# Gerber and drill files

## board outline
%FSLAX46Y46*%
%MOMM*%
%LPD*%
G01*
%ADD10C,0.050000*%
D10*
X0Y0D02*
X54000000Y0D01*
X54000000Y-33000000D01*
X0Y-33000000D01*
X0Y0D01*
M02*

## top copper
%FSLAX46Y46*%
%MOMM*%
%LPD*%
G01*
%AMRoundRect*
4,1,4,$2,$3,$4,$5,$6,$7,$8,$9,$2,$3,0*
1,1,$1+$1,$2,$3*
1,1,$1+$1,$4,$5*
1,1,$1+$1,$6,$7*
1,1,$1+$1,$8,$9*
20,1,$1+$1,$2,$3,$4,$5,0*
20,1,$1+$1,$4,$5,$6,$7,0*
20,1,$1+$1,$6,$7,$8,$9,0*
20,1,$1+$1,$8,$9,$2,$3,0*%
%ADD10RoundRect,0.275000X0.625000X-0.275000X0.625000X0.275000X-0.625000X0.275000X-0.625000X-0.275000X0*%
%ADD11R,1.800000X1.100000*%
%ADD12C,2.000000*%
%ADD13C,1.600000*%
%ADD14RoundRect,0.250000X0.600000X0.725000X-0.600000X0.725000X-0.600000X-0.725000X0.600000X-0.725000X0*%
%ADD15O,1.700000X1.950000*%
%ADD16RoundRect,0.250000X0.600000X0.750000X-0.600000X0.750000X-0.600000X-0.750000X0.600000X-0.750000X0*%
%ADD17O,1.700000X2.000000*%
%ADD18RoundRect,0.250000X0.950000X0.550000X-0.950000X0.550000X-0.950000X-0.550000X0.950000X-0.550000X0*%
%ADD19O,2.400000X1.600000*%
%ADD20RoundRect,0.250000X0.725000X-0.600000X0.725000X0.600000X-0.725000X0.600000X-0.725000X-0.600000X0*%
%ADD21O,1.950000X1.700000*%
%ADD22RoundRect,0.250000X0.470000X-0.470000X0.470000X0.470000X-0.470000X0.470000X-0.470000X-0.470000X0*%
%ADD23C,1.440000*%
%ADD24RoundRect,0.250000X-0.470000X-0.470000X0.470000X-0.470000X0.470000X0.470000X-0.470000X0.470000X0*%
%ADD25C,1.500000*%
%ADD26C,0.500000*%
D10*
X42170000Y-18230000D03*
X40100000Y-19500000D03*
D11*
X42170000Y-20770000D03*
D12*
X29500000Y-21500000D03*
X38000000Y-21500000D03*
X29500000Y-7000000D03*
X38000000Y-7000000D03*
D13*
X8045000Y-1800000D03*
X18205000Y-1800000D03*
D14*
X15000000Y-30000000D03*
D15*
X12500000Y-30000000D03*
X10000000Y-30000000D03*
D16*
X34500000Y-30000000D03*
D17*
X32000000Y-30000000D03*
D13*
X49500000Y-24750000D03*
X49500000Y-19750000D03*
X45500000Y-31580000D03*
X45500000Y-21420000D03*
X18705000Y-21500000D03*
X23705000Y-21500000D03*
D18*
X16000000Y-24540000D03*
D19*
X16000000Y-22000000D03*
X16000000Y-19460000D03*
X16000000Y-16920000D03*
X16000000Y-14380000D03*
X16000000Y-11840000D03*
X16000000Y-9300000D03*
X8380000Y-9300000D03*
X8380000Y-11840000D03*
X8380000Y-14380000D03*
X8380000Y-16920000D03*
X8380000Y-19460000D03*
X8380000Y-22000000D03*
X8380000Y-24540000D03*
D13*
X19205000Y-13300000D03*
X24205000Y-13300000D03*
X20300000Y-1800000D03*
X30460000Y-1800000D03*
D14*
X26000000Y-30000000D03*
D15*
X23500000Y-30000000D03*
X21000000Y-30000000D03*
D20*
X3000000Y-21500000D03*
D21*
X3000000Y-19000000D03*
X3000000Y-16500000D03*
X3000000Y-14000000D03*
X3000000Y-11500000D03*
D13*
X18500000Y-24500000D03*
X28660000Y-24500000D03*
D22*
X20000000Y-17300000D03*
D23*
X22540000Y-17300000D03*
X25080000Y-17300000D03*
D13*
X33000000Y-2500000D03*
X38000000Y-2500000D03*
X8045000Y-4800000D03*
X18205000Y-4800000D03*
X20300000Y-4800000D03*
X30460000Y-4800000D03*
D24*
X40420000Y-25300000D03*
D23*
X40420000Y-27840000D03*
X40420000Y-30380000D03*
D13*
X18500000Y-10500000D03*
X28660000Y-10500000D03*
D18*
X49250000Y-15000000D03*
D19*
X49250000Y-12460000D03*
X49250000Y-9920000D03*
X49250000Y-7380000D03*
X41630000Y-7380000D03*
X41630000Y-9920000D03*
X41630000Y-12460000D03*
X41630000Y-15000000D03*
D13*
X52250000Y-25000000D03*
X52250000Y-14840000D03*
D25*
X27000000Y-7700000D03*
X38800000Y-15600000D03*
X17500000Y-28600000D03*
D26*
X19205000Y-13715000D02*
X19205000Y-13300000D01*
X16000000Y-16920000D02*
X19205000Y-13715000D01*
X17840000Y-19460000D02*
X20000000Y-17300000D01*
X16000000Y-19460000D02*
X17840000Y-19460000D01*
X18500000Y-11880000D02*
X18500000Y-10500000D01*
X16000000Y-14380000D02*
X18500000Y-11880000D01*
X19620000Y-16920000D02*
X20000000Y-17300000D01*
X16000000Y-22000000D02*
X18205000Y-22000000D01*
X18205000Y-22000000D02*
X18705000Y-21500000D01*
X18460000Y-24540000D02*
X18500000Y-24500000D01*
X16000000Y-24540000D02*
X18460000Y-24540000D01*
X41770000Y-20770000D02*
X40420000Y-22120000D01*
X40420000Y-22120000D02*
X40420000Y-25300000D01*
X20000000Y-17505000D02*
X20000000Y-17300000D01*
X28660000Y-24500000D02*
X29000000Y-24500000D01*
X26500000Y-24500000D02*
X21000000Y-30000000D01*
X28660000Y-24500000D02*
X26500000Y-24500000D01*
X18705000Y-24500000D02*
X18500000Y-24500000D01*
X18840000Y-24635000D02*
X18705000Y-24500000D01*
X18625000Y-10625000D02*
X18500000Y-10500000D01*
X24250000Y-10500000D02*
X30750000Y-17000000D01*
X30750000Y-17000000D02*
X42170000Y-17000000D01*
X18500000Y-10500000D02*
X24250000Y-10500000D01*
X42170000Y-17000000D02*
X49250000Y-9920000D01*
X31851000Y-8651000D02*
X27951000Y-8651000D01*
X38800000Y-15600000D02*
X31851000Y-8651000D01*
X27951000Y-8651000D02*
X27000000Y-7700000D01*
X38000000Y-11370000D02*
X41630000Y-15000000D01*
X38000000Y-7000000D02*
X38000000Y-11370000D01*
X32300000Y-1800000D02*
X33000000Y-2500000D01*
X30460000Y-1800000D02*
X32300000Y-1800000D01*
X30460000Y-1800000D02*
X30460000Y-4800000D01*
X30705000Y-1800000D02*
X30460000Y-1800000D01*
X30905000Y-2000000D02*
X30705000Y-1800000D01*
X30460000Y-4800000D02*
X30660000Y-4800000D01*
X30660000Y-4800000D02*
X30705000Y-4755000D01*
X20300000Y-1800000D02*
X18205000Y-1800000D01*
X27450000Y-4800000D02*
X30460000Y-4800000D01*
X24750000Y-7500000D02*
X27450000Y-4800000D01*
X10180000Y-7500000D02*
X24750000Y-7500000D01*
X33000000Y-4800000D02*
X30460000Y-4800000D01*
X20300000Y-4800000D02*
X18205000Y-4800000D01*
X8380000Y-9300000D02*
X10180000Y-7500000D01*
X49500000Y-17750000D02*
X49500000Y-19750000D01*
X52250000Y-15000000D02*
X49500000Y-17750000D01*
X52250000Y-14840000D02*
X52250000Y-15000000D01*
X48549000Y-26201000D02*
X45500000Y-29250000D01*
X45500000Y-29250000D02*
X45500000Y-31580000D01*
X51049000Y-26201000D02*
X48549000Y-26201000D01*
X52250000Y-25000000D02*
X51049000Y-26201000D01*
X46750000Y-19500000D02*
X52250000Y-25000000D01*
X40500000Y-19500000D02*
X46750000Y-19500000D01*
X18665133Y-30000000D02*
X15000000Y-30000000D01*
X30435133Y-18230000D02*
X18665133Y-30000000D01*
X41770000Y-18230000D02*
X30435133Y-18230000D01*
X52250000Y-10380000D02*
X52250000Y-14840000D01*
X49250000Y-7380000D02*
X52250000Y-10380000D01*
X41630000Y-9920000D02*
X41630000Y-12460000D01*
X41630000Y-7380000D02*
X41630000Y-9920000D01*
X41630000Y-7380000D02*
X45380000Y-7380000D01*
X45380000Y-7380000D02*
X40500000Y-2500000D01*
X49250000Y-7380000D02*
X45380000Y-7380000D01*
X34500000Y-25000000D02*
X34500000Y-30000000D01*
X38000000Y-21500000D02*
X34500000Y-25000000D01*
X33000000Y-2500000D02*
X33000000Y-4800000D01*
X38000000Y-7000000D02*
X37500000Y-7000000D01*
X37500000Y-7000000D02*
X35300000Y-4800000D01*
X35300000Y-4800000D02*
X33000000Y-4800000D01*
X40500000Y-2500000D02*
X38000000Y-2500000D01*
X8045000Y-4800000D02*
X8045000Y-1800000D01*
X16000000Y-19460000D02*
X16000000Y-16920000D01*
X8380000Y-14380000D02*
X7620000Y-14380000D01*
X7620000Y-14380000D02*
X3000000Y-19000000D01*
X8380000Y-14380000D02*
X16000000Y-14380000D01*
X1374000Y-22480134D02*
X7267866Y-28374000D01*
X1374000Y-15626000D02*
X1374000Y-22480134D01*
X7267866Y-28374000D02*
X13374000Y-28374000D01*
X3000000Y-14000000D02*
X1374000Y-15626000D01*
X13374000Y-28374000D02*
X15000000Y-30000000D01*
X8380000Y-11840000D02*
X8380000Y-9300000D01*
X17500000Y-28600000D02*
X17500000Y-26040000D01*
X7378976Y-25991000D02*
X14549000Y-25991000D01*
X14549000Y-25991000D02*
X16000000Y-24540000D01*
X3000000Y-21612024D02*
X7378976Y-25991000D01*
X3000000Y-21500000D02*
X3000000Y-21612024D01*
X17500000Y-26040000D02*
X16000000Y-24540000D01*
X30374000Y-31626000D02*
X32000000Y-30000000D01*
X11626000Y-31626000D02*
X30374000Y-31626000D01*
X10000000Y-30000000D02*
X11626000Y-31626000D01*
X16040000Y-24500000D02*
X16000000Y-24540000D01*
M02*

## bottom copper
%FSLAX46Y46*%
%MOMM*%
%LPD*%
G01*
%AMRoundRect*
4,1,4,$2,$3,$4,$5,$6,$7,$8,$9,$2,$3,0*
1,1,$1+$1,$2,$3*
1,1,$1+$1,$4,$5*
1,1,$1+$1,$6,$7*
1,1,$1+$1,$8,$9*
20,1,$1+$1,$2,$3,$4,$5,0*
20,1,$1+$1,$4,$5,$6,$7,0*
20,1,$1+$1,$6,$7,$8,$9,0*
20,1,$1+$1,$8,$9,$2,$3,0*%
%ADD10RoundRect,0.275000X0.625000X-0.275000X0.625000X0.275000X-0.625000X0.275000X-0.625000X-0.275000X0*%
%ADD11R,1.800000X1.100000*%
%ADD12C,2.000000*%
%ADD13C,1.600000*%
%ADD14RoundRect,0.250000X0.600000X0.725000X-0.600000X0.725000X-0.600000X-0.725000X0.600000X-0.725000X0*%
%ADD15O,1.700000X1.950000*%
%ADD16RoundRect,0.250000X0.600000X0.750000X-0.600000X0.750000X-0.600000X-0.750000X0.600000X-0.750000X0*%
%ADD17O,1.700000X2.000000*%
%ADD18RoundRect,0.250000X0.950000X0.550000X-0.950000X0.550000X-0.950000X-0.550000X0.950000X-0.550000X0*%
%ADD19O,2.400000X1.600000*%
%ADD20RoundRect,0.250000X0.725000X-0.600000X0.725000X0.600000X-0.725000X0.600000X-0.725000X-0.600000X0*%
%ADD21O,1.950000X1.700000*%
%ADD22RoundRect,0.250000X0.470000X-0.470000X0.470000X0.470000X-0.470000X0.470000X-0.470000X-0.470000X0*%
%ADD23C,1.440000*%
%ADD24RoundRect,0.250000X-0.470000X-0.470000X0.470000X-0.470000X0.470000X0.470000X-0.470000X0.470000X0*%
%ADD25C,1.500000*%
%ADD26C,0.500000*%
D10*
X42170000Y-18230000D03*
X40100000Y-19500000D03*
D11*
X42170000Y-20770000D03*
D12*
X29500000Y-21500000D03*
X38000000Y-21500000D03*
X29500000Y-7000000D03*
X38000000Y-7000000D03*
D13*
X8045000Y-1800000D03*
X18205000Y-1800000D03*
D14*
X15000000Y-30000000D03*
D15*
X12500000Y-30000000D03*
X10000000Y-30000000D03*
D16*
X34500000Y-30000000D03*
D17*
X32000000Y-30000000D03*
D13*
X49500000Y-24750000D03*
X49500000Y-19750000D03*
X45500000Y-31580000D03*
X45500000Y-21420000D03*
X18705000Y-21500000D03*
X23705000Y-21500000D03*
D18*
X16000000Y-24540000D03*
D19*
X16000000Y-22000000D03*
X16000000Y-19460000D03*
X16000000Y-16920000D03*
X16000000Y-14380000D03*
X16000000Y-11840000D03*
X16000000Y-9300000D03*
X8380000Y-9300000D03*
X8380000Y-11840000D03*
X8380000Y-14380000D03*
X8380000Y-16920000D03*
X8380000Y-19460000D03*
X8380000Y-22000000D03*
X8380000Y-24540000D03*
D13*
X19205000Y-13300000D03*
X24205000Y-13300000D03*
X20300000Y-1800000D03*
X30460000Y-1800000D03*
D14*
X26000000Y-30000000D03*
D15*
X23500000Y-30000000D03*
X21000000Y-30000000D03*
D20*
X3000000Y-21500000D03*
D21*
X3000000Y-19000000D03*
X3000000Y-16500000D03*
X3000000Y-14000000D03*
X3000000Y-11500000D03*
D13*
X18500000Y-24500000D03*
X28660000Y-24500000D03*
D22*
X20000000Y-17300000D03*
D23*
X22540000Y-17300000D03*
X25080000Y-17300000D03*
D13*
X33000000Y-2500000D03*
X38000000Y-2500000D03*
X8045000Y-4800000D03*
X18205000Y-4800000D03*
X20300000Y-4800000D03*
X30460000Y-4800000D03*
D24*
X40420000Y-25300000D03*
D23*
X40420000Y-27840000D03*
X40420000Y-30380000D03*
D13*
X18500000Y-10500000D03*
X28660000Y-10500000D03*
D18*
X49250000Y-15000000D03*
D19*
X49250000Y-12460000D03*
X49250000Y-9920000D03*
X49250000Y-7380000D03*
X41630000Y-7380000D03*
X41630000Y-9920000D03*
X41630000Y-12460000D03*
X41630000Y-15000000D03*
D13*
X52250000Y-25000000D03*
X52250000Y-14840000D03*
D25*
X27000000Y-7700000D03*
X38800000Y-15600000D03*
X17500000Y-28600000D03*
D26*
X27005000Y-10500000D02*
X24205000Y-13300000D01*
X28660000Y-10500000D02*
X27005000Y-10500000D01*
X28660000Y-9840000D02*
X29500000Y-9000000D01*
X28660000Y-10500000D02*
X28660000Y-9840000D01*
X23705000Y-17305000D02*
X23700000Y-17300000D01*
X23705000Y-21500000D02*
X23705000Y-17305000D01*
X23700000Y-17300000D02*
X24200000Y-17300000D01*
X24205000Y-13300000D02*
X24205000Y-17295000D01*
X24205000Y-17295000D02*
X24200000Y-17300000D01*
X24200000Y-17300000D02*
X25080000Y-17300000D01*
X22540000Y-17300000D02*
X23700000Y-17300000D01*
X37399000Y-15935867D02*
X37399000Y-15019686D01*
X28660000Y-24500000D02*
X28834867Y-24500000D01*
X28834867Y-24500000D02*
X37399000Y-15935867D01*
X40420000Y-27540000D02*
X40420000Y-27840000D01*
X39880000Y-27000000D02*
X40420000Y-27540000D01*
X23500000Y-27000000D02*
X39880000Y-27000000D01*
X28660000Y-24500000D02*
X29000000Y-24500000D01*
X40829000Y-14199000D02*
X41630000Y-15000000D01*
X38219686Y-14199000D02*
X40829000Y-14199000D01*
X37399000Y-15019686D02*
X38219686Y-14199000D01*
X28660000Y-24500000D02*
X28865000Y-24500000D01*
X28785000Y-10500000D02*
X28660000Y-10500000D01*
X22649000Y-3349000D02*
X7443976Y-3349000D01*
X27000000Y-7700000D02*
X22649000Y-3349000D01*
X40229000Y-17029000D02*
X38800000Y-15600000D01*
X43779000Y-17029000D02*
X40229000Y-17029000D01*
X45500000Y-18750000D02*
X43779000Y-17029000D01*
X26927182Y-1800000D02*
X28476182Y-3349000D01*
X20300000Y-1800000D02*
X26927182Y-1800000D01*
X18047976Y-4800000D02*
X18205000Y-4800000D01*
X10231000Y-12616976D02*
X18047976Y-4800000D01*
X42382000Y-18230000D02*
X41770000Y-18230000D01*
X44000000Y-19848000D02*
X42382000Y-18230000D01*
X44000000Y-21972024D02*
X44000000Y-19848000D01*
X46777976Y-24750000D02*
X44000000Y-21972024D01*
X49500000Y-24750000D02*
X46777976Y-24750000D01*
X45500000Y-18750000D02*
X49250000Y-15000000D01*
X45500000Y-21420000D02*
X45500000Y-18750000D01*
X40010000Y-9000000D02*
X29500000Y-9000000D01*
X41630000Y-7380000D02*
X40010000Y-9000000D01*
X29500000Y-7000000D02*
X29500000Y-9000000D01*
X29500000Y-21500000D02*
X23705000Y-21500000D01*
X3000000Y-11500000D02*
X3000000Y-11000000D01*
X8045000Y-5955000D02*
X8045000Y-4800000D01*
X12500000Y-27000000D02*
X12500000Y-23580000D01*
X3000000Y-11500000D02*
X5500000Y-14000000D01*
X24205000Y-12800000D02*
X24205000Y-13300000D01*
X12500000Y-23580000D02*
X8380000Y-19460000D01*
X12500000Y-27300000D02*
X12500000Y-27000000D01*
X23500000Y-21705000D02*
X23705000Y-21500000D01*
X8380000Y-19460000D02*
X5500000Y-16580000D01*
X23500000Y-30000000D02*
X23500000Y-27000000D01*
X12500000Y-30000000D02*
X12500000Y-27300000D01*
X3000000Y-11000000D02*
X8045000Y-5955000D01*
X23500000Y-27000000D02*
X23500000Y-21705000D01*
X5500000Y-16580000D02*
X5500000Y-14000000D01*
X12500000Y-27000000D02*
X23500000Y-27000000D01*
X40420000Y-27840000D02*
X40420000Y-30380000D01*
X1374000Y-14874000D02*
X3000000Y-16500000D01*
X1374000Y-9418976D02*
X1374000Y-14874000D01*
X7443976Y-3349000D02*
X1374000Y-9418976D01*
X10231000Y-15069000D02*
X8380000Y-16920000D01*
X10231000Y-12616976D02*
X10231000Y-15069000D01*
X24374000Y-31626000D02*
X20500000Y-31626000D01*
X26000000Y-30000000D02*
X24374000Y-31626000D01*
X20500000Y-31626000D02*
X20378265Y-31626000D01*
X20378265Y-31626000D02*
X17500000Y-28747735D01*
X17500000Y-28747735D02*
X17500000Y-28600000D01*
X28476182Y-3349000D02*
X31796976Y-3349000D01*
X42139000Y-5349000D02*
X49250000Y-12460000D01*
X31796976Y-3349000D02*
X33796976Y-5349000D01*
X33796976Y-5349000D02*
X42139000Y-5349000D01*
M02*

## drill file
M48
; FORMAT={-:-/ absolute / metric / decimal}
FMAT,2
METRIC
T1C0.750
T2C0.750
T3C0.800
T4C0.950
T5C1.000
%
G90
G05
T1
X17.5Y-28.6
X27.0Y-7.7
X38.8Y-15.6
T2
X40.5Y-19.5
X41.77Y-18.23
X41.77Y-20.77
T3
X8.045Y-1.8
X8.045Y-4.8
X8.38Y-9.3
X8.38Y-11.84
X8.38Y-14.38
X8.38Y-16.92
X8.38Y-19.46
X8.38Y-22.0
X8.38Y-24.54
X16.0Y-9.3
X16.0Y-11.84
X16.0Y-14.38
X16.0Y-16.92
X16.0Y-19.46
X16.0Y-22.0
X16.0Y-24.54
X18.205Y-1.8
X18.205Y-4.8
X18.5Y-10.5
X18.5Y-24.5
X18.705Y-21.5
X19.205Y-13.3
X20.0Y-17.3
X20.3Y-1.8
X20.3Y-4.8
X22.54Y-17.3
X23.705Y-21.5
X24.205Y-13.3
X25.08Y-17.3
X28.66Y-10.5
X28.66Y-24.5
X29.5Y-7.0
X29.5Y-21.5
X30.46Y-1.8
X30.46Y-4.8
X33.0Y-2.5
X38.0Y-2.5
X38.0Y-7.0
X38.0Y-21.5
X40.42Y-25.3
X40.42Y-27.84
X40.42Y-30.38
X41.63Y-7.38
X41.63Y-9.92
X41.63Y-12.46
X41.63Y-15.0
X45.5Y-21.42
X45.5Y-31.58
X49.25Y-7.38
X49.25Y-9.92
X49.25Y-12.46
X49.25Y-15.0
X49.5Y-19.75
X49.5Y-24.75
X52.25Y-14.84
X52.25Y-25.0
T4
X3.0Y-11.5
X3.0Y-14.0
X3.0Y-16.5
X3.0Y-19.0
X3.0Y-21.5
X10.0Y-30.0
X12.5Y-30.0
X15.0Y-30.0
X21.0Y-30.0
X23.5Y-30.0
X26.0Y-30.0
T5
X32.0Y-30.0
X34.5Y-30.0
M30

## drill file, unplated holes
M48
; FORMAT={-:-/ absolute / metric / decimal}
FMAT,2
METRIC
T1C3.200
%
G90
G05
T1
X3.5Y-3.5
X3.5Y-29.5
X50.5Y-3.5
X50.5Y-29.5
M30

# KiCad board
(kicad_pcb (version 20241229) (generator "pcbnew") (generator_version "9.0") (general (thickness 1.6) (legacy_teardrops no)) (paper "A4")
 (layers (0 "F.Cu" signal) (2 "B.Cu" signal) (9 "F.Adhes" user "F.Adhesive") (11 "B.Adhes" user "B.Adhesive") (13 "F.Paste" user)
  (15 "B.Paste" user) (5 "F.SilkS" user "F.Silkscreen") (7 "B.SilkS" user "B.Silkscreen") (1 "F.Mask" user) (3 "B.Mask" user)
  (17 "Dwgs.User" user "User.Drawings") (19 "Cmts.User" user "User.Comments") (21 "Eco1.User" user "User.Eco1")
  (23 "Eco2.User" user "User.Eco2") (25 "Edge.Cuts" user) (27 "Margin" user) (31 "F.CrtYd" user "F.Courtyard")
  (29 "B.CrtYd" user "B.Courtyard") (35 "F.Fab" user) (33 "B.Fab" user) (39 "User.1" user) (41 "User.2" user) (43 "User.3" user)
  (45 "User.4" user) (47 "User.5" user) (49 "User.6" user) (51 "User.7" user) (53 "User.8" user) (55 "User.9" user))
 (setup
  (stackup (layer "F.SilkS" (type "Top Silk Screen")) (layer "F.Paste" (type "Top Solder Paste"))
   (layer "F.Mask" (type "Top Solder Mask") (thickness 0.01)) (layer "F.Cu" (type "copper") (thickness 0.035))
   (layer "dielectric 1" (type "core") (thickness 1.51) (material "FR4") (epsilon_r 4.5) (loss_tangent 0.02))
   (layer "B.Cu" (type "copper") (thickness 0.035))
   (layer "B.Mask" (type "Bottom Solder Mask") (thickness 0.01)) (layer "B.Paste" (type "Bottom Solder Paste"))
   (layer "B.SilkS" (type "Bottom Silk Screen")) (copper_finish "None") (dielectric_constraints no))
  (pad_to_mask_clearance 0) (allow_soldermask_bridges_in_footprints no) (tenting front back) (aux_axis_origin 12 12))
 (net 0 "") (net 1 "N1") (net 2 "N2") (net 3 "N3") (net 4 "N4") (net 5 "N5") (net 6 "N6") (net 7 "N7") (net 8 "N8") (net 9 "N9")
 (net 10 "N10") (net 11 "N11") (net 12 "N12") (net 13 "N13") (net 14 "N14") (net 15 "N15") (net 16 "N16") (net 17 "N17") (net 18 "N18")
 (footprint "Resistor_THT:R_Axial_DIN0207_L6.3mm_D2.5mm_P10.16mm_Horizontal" (layer "F.Cu") (at 20.045 13.8)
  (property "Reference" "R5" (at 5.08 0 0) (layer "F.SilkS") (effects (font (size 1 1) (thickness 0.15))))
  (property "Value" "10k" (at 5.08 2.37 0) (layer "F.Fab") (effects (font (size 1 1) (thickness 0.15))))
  (pad "1" thru_hole circle (at 0 0) (size 1.6 1.6) (drill 0.8) (layers "*.Cu" "*.Mask") (remove_unused_layers no) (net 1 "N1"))
  (pad "2" thru_hole circle (at 10.16 0) (size 1.6 1.6) (drill 0.8) (layers "*.Cu" "*.Mask") (remove_unused_layers no) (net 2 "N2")))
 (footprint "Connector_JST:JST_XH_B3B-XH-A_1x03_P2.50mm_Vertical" (layer "F.Cu") (at 27 42 180)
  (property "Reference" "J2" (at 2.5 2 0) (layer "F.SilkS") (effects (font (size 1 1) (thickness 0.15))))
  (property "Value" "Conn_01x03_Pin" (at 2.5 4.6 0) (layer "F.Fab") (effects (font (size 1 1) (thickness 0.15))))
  (pad "1" thru_hole roundrect (at 0 0 180) (size 1.7 1.95) (drill 0.95) (layers "*.Cu" "*.Mask") (remove_unused_layers no)
   (roundrect_rratio 0.147059) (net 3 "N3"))
  (pad "2" thru_hole oval (at 2.5 0 180) (size 1.7 1.95) (drill 0.95) (layers "*.Cu" "*.Mask") (remove_unused_layers no) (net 1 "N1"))
  (pad "3" thru_hole oval (at 5 0 180) (size 1.7 1.95) (drill 0.95) (layers "*.Cu" "*.Mask") (remove_unused_layers no) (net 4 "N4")))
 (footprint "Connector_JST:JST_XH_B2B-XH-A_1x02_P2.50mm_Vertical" (layer "F.Cu") (at 46.5 42 180)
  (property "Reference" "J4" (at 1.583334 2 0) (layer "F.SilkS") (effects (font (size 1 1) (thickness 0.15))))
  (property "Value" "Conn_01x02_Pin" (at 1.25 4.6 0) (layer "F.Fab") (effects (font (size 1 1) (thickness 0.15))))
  (pad "1" thru_hole roundrect (at 0 0 180) (size 1.7 2) (drill 1) (layers "*.Cu" "*.Mask") (remove_unused_layers no)
   (roundrect_rratio 0.147059) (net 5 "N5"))
  (pad "2" thru_hole oval (at 2.5 0 180) (size 1.7 2) (drill 1) (layers "*.Cu" "*.Mask") (remove_unused_layers no) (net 4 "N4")))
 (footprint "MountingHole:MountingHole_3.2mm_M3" (layer "F.Cu") (at 15.5 41.5 90)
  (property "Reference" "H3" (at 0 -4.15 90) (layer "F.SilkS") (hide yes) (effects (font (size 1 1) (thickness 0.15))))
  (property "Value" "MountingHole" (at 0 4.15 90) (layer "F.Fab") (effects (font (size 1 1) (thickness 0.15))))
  (pad "" np_thru_hole circle (at 0 0 90) (size 3.2 3.2) (drill 3.2) (layers "*.Cu" "*.Mask")))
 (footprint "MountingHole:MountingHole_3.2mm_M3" (layer "F.Cu") (at 62.5 15.5 90)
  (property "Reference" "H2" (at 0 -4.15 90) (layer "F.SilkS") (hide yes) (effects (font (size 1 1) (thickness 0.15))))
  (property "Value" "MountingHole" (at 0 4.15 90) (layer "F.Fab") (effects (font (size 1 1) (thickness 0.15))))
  (pad "" np_thru_hole circle (at 0 0 90) (size 3.2 3.2) (drill 3.2) (layers "*.Cu" "*.Mask")))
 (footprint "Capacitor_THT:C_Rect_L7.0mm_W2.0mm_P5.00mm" (layer "F.Cu") (at 61.5 36.75 90)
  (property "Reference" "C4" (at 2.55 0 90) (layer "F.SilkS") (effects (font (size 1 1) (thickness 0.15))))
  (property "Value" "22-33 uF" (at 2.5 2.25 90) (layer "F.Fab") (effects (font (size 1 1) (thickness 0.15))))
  (pad "1" thru_hole circle (at 0 0 90) (size 1.6 1.6) (drill 0.8) (layers "*.Cu" "*.Mask") (remove_unused_layers no) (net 3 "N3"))
  (pad "2" thru_hole circle (at 5 0 90) (size 1.6 1.6) (drill 0.8) (layers "*.Cu" "*.Mask") (remove_unused_layers no) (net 1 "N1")))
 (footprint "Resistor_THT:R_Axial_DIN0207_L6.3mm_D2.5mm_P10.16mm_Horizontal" (layer "F.Cu") (at 57.5 43.58 90)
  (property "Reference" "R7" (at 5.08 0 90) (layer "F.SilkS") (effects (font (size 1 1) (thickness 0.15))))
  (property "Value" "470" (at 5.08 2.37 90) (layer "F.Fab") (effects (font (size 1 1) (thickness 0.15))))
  (pad "1" thru_hole circle (at 0 0 90) (size 1.6 1.6) (drill 0.8) (layers "*.Cu" "*.Mask") (remove_unused_layers no) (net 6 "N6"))
  (pad "2" thru_hole circle (at 10.16 0 90) (size 1.6 1.6) (drill 0.8) (layers "*.Cu" "*.Mask") (remove_unused_layers no) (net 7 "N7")))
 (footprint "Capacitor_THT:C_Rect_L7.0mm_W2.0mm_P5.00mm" (layer "F.Cu") (at 30.705 33.5)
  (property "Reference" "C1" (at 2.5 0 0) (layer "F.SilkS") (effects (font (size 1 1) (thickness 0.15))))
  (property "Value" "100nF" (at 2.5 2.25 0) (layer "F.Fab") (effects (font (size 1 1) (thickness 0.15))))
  (pad "1" thru_hole circle (at 0 0) (size 1.6 1.6) (drill 0.8) (layers "*.Cu" "*.Mask") (remove_unused_layers no) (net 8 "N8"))
  (pad "2" thru_hole circle (at 5 0) (size 1.6 1.6) (drill 0.8) (layers "*.Cu" "*.Mask") (remove_unused_layers no) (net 1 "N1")))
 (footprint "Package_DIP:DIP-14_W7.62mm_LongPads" (layer "F.Cu") (at 28 36.54 180)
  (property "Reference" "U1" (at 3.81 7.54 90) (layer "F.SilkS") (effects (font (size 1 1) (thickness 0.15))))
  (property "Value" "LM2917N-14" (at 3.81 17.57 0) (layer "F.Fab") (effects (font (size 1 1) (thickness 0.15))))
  (pad "1" thru_hole roundrect (at 0 0 180) (size 2.4 1.6) (drill 0.8) (layers "*.Cu" "*.Mask") (remove_unused_layers no)
   (roundrect_rratio 0.15625) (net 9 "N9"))
  (pad "2" thru_hole oval (at 0 2.54 180) (size 2.4 1.6) (drill 0.8) (layers "*.Cu" "*.Mask") (remove_unused_layers no) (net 8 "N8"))
  (pad "3" thru_hole oval (at 0 5.08 180) (size 2.4 1.6) (drill 0.8) (layers "*.Cu" "*.Mask") (remove_unused_layers no) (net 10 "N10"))
  (pad "4" thru_hole oval (at 0 7.62 180) (size 2.4 1.6) (drill 0.8) (layers "*.Cu" "*.Mask") (remove_unused_layers no) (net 10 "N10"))
  (pad "5" thru_hole oval (at 0 10.16 180) (size 2.4 1.6) (drill 0.8) (layers "*.Cu" "*.Mask") (remove_unused_layers no) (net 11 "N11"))
  (pad "6" thru_hole oval (at 0 12.7 180) (size 2.4 1.6) (drill 0.8) (layers "*.Cu" "*.Mask") (remove_unused_layers no) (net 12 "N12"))
  (pad "7" thru_hole oval (at 0 15.24 180) (size 2.4 1.6) (drill 0.8) (layers "*.Cu" "*.Mask") (remove_unused_layers no) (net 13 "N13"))
  (pad "8" thru_hole oval (at 7.62 15.24 180) (size 2.4 1.6) (drill 0.8) (layers "*.Cu" "*.Mask") (remove_unused_layers no) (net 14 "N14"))
  (pad "9" thru_hole oval (at 7.62 12.7 180) (size 2.4 1.6) (drill 0.8) (layers "*.Cu" "*.Mask") (remove_unused_layers no) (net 14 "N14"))
  (pad "10" thru_hole oval (at 7.62 10.16 180) (size 2.4 1.6) (drill 0.8) (layers "*.Cu" "*.Mask") (remove_unused_layers no) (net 11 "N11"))
  (pad "11" thru_hole oval (at 7.62 7.62 180) (size 2.4 1.6) (drill 0.8) (layers "*.Cu" "*.Mask") (remove_unused_layers no) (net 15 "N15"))
  (pad "12" thru_hole oval (at 7.62 5.08 180) (size 2.4 1.6) (drill 0.8) (layers "*.Cu" "*.Mask") (remove_unused_layers no) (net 1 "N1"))
  (pad "13" thru_hole oval (at 7.62 2.54 180) (size 2.4 1.6) (drill 0.8) (layers "*.Cu" "*.Mask") (remove_unused_layers no) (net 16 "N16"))
  (pad "14" thru_hole oval (at 7.62 0 180) (size 2.4 1.6) (drill 0.8) (layers "*.Cu" "*.Mask") (remove_unused_layers no) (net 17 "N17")))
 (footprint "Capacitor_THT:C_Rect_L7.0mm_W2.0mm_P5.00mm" (layer "F.Cu") (at 31.205 25.3)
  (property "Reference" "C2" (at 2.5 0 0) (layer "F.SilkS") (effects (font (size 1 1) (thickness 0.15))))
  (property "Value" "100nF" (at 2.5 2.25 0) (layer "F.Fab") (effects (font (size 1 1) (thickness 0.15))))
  (pad "1" thru_hole circle (at 0 0) (size 1.6 1.6) (drill 0.8) (layers "*.Cu" "*.Mask") (remove_unused_layers no) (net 10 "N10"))
  (pad "2" thru_hole circle (at 5 0) (size 1.6 1.6) (drill 0.8) (layers "*.Cu" "*.Mask") (remove_unused_layers no) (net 1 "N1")))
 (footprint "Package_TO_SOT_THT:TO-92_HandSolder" (layer "F.Cu") (at 53.77 32.77 90)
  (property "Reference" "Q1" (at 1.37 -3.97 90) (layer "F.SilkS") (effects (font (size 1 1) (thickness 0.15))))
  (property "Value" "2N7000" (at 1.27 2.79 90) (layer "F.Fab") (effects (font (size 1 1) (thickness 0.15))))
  (pad "1" thru_hole rect (at 0 0 90) (size 1.1 1.8) (drill 0.75 (offset 0 0.4)) (layers "*.Cu" "*.Mask") (remove_unused_layers no)
   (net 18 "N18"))
  (pad "2" thru_hole roundrect (at 1.27 -1.27 90) (size 1.1 1.8) (drill 0.75 (offset 0 -0.4)) (layers "*.Cu" "*.Mask")
   (remove_unused_layers no) (roundrect_rratio 0.25) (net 6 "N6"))
  (pad "3" thru_hole roundrect (at 2.54 0 90) (size 1.1 1.8) (drill 0.75 (offset 0 0.4)) (layers "*.Cu" "*.Mask") (remove_unused_layers no)
   (roundrect_rratio 0.25) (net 3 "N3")))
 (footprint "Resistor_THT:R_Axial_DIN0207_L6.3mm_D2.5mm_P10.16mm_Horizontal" (layer "F.Cu") (at 32.3 13.8)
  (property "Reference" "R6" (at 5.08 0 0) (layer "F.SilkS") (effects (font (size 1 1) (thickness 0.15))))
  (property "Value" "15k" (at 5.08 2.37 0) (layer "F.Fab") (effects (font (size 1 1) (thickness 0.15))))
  (pad "1" thru_hole circle (at 0 0) (size 1.6 1.6) (drill 0.8) (layers "*.Cu" "*.Mask") (remove_unused_layers no) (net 2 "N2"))
  (pad "2" thru_hole circle (at 10.16 0) (size 1.6 1.6) (drill 0.8) (layers "*.Cu" "*.Mask") (remove_unused_layers no) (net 14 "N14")))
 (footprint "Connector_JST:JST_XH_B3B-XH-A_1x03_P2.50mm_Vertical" (layer "F.Cu") (at 38 42 180)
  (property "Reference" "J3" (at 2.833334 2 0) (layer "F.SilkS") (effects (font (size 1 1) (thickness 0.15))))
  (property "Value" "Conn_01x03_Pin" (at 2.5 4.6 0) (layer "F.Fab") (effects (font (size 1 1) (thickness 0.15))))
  (pad "1" thru_hole roundrect (at 0 0 180) (size 1.7 1.95) (drill 0.95) (layers "*.Cu" "*.Mask") (remove_unused_layers no)
   (roundrect_rratio 0.147059) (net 9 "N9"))
  (pad "2" thru_hole oval (at 2.5 0 180) (size 1.7 1.95) (drill 0.95) (layers "*.Cu" "*.Mask") (remove_unused_layers no) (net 1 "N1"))
  (pad "3" thru_hole oval (at 5 0 180) (size 1.7 1.95) (drill 0.95) (layers "*.Cu" "*.Mask") (remove_unused_layers no) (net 14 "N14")))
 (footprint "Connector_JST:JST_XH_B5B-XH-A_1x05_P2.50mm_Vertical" (layer "F.Cu") (at 15 33.5 90)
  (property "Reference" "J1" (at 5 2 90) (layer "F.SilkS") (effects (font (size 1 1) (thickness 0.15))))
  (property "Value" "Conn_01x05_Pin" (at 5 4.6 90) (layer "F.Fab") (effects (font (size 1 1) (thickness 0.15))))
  (pad "1" thru_hole roundrect (at 0 0 90) (size 1.7 1.95) (drill 0.95) (layers "*.Cu" "*.Mask") (remove_unused_layers no)
   (roundrect_rratio 0.147059) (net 9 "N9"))
  (pad "2" thru_hole oval (at 2.5 0 90) (size 1.7 1.95) (drill 0.95) (layers "*.Cu" "*.Mask") (remove_unused_layers no) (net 11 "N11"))
  (pad "3" thru_hole oval (at 5 0 90) (size 1.7 1.95) (drill 0.95) (layers "*.Cu" "*.Mask") (remove_unused_layers no) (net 7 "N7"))
  (pad "4" thru_hole oval (at 7.5 0 90) (size 1.7 1.95) (drill 0.95) (layers "*.Cu" "*.Mask") (remove_unused_layers no) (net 3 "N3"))
  (pad "5" thru_hole oval (at 10 0 90) (size 1.7 1.95) (drill 0.95) (layers "*.Cu" "*.Mask") (remove_unused_layers no) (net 1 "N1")))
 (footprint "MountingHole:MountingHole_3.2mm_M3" (layer "F.Cu") (at 62.5 41.5 90)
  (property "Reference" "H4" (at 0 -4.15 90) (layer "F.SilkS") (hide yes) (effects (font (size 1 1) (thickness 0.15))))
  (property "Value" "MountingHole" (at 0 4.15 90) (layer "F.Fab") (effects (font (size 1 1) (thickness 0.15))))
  (pad "" np_thru_hole circle (at 0 0 90) (size 3.2 3.2) (drill 3.2) (layers "*.Cu" "*.Mask")))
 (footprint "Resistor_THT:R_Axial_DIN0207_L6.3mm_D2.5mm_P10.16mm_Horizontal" (layer "F.Cu") (at 30.5 36.5)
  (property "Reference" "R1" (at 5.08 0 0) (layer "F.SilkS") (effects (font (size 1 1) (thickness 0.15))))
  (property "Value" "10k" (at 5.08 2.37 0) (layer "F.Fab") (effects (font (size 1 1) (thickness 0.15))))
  (pad "1" thru_hole circle (at 0 0) (size 1.6 1.6) (drill 0.8) (layers "*.Cu" "*.Mask") (remove_unused_layers no) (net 9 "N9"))
  (pad "2" thru_hole circle (at 10.16 0) (size 1.6 1.6) (drill 0.8) (layers "*.Cu" "*.Mask") (remove_unused_layers no) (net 14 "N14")))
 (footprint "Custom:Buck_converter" (layer "F.Cu") (at 45.75 26.25 90)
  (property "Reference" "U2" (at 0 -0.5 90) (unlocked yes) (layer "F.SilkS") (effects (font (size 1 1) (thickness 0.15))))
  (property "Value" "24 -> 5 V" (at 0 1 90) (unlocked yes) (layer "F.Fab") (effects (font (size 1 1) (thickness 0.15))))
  (pad "1" thru_hole circle (at -7.25 -4.25 90) (size 2 2) (drill 0.8) (layers "*.Cu" "*.Mask") (remove_unused_layers no) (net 1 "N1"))
  (pad "2" thru_hole circle (at -7.25 4.25 90) (size 2 2) (drill 0.8) (layers "*.Cu" "*.Mask") (remove_unused_layers no) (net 5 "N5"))
  (pad "3" thru_hole circle (at 7.25 -4.25 90) (size 2 2) (drill 0.8) (layers "*.Cu" "*.Mask") (remove_unused_layers no) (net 1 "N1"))
  (pad "4" thru_hole circle (at 7.25 4.25 90) (size 2 2) (drill 0.8) (layers "*.Cu" "*.Mask") (remove_unused_layers no) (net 14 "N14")))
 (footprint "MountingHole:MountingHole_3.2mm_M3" (layer "F.Cu") (at 15.5 15.5 90)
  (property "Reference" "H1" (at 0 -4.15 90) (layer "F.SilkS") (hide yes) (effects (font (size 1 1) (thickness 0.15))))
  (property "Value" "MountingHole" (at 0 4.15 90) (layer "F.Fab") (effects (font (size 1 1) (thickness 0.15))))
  (pad "" np_thru_hole circle (at 0 0 90) (size 3.2 3.2) (drill 3.2) (layers "*.Cu" "*.Mask")))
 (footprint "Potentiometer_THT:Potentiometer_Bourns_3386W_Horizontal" (layer "F.Cu") (at 32 29.3)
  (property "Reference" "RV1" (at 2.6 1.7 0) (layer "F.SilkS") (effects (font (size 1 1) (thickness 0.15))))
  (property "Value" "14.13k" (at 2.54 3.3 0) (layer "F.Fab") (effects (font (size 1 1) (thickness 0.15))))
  (pad "1" thru_hole roundrect (at 0 0 90) (size 1.44 1.44) (drill 0.8) (layers "*.Cu" "*.Mask") (remove_unused_layers no)
   (roundrect_rratio 0.1736111111) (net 10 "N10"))
  (pad "2" thru_hole circle (at 2.54 0 90) (size 1.44 1.44) (drill 0.8) (layers "*.Cu" "*.Mask") (remove_unused_layers no) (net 1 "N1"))
  (pad "3" thru_hole circle (at 5.08 0 90) (size 1.44 1.44) (drill 0.8) (layers "*.Cu" "*.Mask") (remove_unused_layers no) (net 1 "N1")))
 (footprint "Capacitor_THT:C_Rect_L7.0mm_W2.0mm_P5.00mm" (layer "F.Cu") (at 45 14.5)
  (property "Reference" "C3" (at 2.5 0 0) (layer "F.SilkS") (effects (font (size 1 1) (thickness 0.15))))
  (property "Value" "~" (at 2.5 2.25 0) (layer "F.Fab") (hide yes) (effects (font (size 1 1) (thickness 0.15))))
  (pad "1" thru_hole circle (at 0 0) (size 1.6 1.6) (drill 0.8) (layers "*.Cu" "*.Mask") (remove_unused_layers no) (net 14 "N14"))
  (pad "2" thru_hole circle (at 5 0) (size 1.6 1.6) (drill 0.8) (layers "*.Cu" "*.Mask") (remove_unused_layers no) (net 1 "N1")))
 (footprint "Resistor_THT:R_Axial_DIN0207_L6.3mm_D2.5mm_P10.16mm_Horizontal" (layer "F.Cu") (at 20.045 16.8)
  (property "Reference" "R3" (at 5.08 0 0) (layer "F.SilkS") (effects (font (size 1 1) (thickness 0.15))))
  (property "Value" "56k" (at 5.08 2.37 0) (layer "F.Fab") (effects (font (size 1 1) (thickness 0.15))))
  (pad "1" thru_hole circle (at 0 0) (size 1.6 1.6) (drill 0.8) (layers "*.Cu" "*.Mask") (remove_unused_layers no) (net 1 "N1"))
  (pad "2" thru_hole circle (at 10.16 0) (size 1.6 1.6) (drill 0.8) (layers "*.Cu" "*.Mask") (remove_unused_layers no) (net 15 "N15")))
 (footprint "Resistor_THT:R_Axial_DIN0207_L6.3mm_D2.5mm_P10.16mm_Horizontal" (layer "F.Cu") (at 32.3 16.8)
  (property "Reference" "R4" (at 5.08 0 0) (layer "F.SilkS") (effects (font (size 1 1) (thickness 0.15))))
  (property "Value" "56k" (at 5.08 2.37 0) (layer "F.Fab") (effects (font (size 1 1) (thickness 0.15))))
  (pad "1" thru_hole circle (at 0 0) (size 1.6 1.6) (drill 0.8) (layers "*.Cu" "*.Mask") (remove_unused_layers no) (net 15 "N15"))
  (pad "2" thru_hole circle (at 10.16 0) (size 1.6 1.6) (drill 0.8) (layers "*.Cu" "*.Mask") (remove_unused_layers no) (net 14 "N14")))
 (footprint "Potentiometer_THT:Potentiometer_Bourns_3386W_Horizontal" (layer "F.Cu") (at 52.42 37.3 -90)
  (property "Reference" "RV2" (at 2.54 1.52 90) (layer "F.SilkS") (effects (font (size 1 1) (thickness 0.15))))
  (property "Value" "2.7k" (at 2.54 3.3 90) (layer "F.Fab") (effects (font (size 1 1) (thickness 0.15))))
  (pad "1" thru_hole roundrect (at 0 0) (size 1.44 1.44) (drill 0.8) (layers "*.Cu" "*.Mask") (remove_unused_layers no)
   (roundrect_rratio 0.1736111111) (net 18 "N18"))
  (pad "2" thru_hole circle (at 2.54 0) (size 1.44 1.44) (drill 0.8) (layers "*.Cu" "*.Mask") (remove_unused_layers no) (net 1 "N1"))
  (pad "3" thru_hole circle (at 5.08 0) (size 1.44 1.44) (drill 0.8) (layers "*.Cu" "*.Mask") (remove_unused_layers no) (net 1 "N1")))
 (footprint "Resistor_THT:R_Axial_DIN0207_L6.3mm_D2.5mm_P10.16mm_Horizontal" (layer "F.Cu") (at 30.5 22.5)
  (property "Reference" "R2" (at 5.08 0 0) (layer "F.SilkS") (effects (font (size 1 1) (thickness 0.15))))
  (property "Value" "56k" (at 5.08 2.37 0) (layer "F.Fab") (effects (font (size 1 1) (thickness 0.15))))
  (pad "1" thru_hole circle (at 0 0) (size 1.6 1.6) (drill 0.8) (layers "*.Cu" "*.Mask") (remove_unused_layers no) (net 11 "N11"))
  (pad "2" thru_hole circle (at 10.16 0) (size 1.6 1.6) (drill 0.8) (layers "*.Cu" "*.Mask") (remove_unused_layers no) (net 1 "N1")))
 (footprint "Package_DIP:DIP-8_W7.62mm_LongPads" (layer "F.Cu") (at 61.25 27 180)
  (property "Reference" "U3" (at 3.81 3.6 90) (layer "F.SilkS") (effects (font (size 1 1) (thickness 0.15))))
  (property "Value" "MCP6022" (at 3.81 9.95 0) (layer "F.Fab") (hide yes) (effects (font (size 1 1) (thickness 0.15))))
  (pad "1" thru_hole roundrect (at 0 0 180) (size 2.4 1.6) (drill 0.8) (layers "*.Cu" "*.Mask") (remove_unused_layers no)
   (roundrect_rratio 0.15625) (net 7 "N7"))
  (pad "2" thru_hole oval (at 0 2.54 180) (size 2.4 1.6) (drill 0.8) (layers "*.Cu" "*.Mask") (remove_unused_layers no) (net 2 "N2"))
  (pad "3" thru_hole oval (at 0 5.08 180) (size 2.4 1.6) (drill 0.8) (layers "*.Cu" "*.Mask") (remove_unused_layers no) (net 11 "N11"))
  (pad "4" thru_hole oval (at 0 7.62 180) (size 2.4 1.6) (drill 0.8) (layers "*.Cu" "*.Mask") (remove_unused_layers no) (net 1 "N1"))
  (pad "5" thru_hole oval (at 7.62 7.62 180) (size 2.4 1.6) (drill 0.8) (layers "*.Cu" "*.Mask") (remove_unused_layers no) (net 1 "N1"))
  (pad "6" thru_hole oval (at 7.62 5.08 180) (size 2.4 1.6) (drill 0.8) (layers "*.Cu" "*.Mask") (remove_unused_layers no) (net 1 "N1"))
  (pad "7" thru_hole oval (at 7.62 2.54 180) (size 2.4 1.6) (drill 0.8) (layers "*.Cu" "*.Mask") (remove_unused_layers no) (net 1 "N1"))
  (pad "8" thru_hole oval (at 7.62 0 180) (size 2.4 1.6) (drill 0.8) (layers "*.Cu" "*.Mask") (remove_unused_layers no) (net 14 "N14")))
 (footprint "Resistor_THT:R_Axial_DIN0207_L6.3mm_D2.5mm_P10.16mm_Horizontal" (layer "F.Cu") (at 64.25 37 90)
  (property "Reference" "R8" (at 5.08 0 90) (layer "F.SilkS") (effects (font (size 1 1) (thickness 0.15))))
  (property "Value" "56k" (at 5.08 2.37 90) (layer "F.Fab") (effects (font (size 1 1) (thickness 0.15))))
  (pad "1" thru_hole circle (at 0 0 90) (size 1.6 1.6) (drill 0.8) (layers "*.Cu" "*.Mask") (remove_unused_layers no) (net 6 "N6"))
  (pad "2" thru_hole circle (at 10.16 0 90) (size 1.6 1.6) (drill 0.8) (layers "*.Cu" "*.Mask") (remove_unused_layers no) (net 1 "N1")))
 (gr_rect (start 12 12) (end 66 45) (stroke (width 0.05) (type default)) (fill no) (layer "Edge.Cuts"))
 (segment (start 28 34) (end 30.205 34) (width 0.5) (layer "F.Cu") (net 8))
 (segment (start 30.205 34) (end 30.705 33.5) (width 0.5) (layer "F.Cu") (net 8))
 (segment (start 28 31.46) (end 29.84 31.46) (width 0.5) (layer "F.Cu") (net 10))
 (segment (start 32 29.505) (end 32 29.3) (width 0.5) (layer "F.Cu") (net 10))
 (segment (start 31.62 28.92) (end 32 29.3) (width 0.5) (layer "F.Cu") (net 10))
 (segment (start 28 28.92) (end 31.205 25.715) (width 0.5) (layer "F.Cu") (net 10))
 (segment (start 31.205 25.715) (end 31.205 25.3) (width 0.5) (layer "F.Cu") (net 10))
 (segment (start 28 31.46) (end 28 28.92) (width 0.5) (layer "F.Cu") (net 10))
 (segment (start 29.84 31.46) (end 32 29.3) (width 0.5) (layer "F.Cu") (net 10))
 (segment (start 30.625 22.625) (end 30.5 22.5) (width 0.5) (layer "F.Cu") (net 11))
 (segment (start 42.75 29) (end 54.17 29) (width 0.5) (layer "F.Cu") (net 11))
 (segment (start 28 26.38) (end 30.5 23.88) (width 0.5) (layer "F.Cu") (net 11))
 (segment (start 20.38 26.38) (end 19.62 26.38) (width 0.5) (layer "F.Cu") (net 11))
 (segment (start 30.5 22.5) (end 36.25 22.5) (width 0.5) (layer "F.Cu") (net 11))
 (segment (start 19.62 26.38) (end 15 31) (width 0.5) (layer "F.Cu") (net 11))
 (segment (start 36.25 22.5) (end 42.75 29) (width 0.5) (layer "F.Cu") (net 11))
 (segment (start 54.17 29) (end 61.25 21.92) (width 0.5) (layer "F.Cu") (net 11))
 (segment (start 30.5 23.88) (end 30.5 22.5) (width 0.5) (layer "F.Cu") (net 11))
 (segment (start 20.38 26.38) (end 28 26.38) (width 0.5) (layer "F.Cu") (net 11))
 (segment (start 39.951 20.651) (end 39 19.7) (width 0.5) (layer "F.Cu") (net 7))
 (segment (start 50.8 27.6) (end 43.851 20.651) (width 0.5) (layer "F.Cu") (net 7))
 (segment (start 43.851 20.651) (end 39.951 20.651) (width 0.5) (layer "F.Cu") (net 7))
 (via (at 39 19.7) (size 1.5) (drill 0.75) (layers "F.Cu" "B.Cu") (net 7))
 (via (at 50.8 27.6) (size 1.5) (drill 0.75) (layers "F.Cu" "B.Cu") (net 7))
 (segment (start 13.374 26.874) (end 15 28.5) (width 0.5) (layer "B.Cu") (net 7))
 (segment (start 57.5 30.75) (end 55.779 29.029) (width 0.5) (layer "B.Cu") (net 7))
 (segment (start 34.649 15.349) (end 19.443976 15.349) (width 0.5) (layer "B.Cu") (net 7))
 (segment (start 52.229 29.029) (end 50.8 27.6) (width 0.5) (layer "B.Cu") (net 7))
 (segment (start 55.779 29.029) (end 52.229 29.029) (width 0.5) (layer "B.Cu") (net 7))
 (segment (start 13.374 21.418976) (end 13.374 26.874) (width 0.5) (layer "B.Cu") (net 7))
 (segment (start 19.443976 15.349) (end 13.374 21.418976) (width 0.5) (layer "B.Cu") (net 7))
 (segment (start 39 19.7) (end 34.649 15.349) (width 0.5) (layer "B.Cu") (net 7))
 (segment (start 57.5 30.75) (end 61.25 27) (width 0.5) (layer "B.Cu") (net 7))
 (segment (start 57.5 33.42) (end 57.5 30.75) (width 0.5) (layer "B.Cu") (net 7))
 (segment (start 13.374 34.480134) (end 19.267866 40.374) (width 0.5) (layer "F.Cu") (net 3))
 (segment (start 30.665133 42) (end 27 42) (width 0.5) (layer "F.Cu") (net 3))
 (segment (start 13.374 27.626) (end 13.374 34.480134) (width 0.5) (layer "F.Cu") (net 3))
 (segment (start 42.435133 30.23) (end 30.665133 42) (width 0.5) (layer "F.Cu") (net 3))
 (segment (start 19.267866 40.374) (end 25.374 40.374) (width 0.5) (layer "F.Cu") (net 3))
 (segment (start 53.77 30.23) (end 42.435133 30.23) (width 0.5) (layer "F.Cu") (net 3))
 (segment (start 15 26) (end 13.374 27.626) (width 0.5) (layer "F.Cu") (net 3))
 (segment (start 25.374 40.374) (end 27 42) (width 0.5) (layer "F.Cu") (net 3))
 (segment (start 56 33.972024) (end 56 31.848) (width 0.5) (layer "B.Cu") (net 3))
 (segment (start 54.382 30.23) (end 53.77 30.23) (width 0.5) (layer "B.Cu") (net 3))
 (segment (start 56 31.848) (end 54.382 30.23) (width 0.5) (layer "B.Cu") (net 3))
 (segment (start 58.777976 36.75) (end 56 33.972024) (width 0.5) (layer "B.Cu") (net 3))
 (segment (start 61.5 36.75) (end 58.777976 36.75) (width 0.5) (layer "B.Cu") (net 3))
 (segment (start 61.25 19.38) (end 57.38 19.38) (width 0.5) (layer "F.Cu") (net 1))
 (segment (start 53.63 19.38) (end 53.63 21.92) (width 0.5) (layer "F.Cu") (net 1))
 (segment (start 52.5 14.5) (end 50 14.5) (width 0.5) (layer "F.Cu") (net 1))
 (segment (start 61.5 29.75) (end 61.5 31.75) (width 0.5) (layer "F.Cu") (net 1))
 (segment (start 53.63 19.38) (end 57.38 19.38) (width 0.5) (layer "F.Cu") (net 1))
 (segment (start 57.38 19.38) (end 52.5 14.5) (width 0.5) (layer "F.Cu") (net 1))
 (segment (start 53.63 21.92) (end 53.63 24.46) (width 0.5) (layer "F.Cu") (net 1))
 (segment (start 61.25 19.38) (end 64.25 22.38) (width 0.5) (layer "F.Cu") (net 1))
 (segment (start 64.25 27) (end 61.5 29.75) (width 0.5) (layer "F.Cu") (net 1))
 (segment (start 64.25 26.84) (end 64.25 27) (width 0.5) (layer "F.Cu") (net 1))
 (segment (start 20.045 16.8) (end 20.045 13.8) (width 0.5) (layer "F.Cu") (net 1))
 (segment (start 64.25 22.38) (end 64.25 26.84) (width 0.5) (layer "F.Cu") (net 1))
 (segment (start 15 23.5) (end 15 23) (width 0.5) (layer "B.Cu") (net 1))
 (segment (start 20.045 17.955) (end 20.045 16.8) (width 0.5) (layer "B.Cu") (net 1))
 (segment (start 41.5 19) (end 41.5 21) (width 0.5) (layer "B.Cu") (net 1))
 (segment (start 24.5 39) (end 24.5 35.58) (width 0.5) (layer "B.Cu") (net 1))
 (segment (start 53.63 19.38) (end 52.01 21) (width 0.5) (layer "B.Cu") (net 1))
 (segment (start 39.005 22.5) (end 36.205 25.3) (width 0.5) (layer "B.Cu") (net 1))
 (segment (start 15 23.5) (end 17.5 26) (width 0.5) (layer "B.Cu") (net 1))
 (segment (start 35.705 29.305) (end 35.7 29.3) (width 0.5) (layer "B.Cu") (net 1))
 (segment (start 52.42 39.54) (end 52.42 39.84) (width 0.5) (layer "B.Cu") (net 1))
 (segment (start 35.7 29.3) (end 36.2 29.3) (width 0.5) (layer "B.Cu") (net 1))
 (segment (start 36.205 24.8) (end 36.205 25.3) (width 0.5) (layer "B.Cu") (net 1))
 (segment (start 24.5 35.58) (end 20.38 31.46) (width 0.5) (layer "B.Cu") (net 1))
 (segment (start 24.5 39.3) (end 24.5 39) (width 0.5) (layer "B.Cu") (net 1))
 (segment (start 35.5 33.705) (end 35.705 33.5) (width 0.5) (layer "B.Cu") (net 1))
 (segment (start 40.785 22.5) (end 40.66 22.5) (width 0.5) (layer "B.Cu") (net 1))
 (segment (start 52.01 21) (end 41.5 21) (width 0.5) (layer "B.Cu") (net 1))
 (segment (start 20.38 31.46) (end 17.5 28.58) (width 0.5) (layer "B.Cu") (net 1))
 (segment (start 35.5 42) (end 35.5 39) (width 0.5) (layer "B.Cu") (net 1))
 (segment (start 24.5 42) (end 24.5 39.3) (width 0.5) (layer "B.Cu") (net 1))
 (segment (start 36.205 29.295) (end 36.2 29.3) (width 0.5) (layer "B.Cu") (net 1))
 (segment (start 41.5 33.5) (end 35.705 33.5) (width 0.5) (layer "B.Cu") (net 1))
 (segment (start 15 23) (end 20.045 17.955) (width 0.5) (layer "B.Cu") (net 1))
 (segment (start 40.66 21.84) (end 41.5 21) (width 0.5) (layer "B.Cu") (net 1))
 (segment (start 40.66 22.5) (end 39.005 22.5) (width 0.5) (layer "B.Cu") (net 1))
 (segment (start 35.5 39) (end 35.5 33.705) (width 0.5) (layer "B.Cu") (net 1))
 (segment (start 40.66 22.5) (end 40.66 21.84) (width 0.5) (layer "B.Cu") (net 1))
 (segment (start 35.5 39) (end 51.88 39) (width 0.5) (layer "B.Cu") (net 1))
 (segment (start 17.5 28.58) (end 17.5 26) (width 0.5) (layer "B.Cu") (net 1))
 (segment (start 24.5 39) (end 35.5 39) (width 0.5) (layer "B.Cu") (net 1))
 (segment (start 52.42 39.84) (end 52.42 42.38) (width 0.5) (layer "B.Cu") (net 1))
 (segment (start 36.2 29.3) (end 37.08 29.3) (width 0.5) (layer "B.Cu") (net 1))
 (segment (start 36.205 25.3) (end 36.205 29.295) (width 0.5) (layer "B.Cu") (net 1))
 (segment (start 51.88 39) (end 52.42 39.54) (width 0.5) (layer "B.Cu") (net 1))
 (segment (start 35.705 33.5) (end 35.705 29.305) (width 0.5) (layer "B.Cu") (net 1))
 (segment (start 34.54 29.3) (end 35.7 29.3) (width 0.5) (layer "B.Cu") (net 1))
 (segment (start 20.38 23.84) (end 20.38 21.3) (width 0.5) (layer "F.Cu") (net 14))
 (segment (start 44.3 13.8) (end 45 14.5) (width 0.5) (layer "F.Cu") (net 14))
 (segment (start 50 19) (end 49.5 19) (width 0.5) (layer "F.Cu") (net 14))
 (segment (start 40.66 36.5) (end 38.5 36.5) (width 0.5) (layer "F.Cu") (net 14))
 (segment (start 49.5 19) (end 47.3 16.8) (width 0.5) (layer "F.Cu") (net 14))
 (segment (start 50 19) (end 50 23.37) (width 0.5) (layer "F.Cu") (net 14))
 (segment (start 45 14.5) (end 45 16.8) (width 0.5) (layer "F.Cu") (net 14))
 (segment (start 42.705 13.8) (end 42.46 13.8) (width 0.5) (layer "F.Cu") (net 14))
 (segment (start 47.3 16.8) (end 45 16.8) (width 0.5) (layer "F.Cu") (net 14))
 (segment (start 42.46 13.8) (end 42.46 16.8) (width 0.5) (layer "F.Cu") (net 14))
 (segment (start 42.46 16.8) (end 42.66 16.8) (width 0.5) (layer "F.Cu") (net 14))
 (segment (start 36.75 19.5) (end 39.45 16.8) (width 0.5) (layer "F.Cu") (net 14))
 (segment (start 42.46 13.8) (end 44.3 13.8) (width 0.5) (layer "F.Cu") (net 14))
 (segment (start 42.66 16.8) (end 42.705 16.755) (width 0.5) (layer "F.Cu") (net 14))
 (segment (start 39.45 16.8) (end 42.46 16.8) (width 0.5) (layer "F.Cu") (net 14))
 (segment (start 40.66 36.5) (end 41 36.5) (width 0.5) (layer "F.Cu") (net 14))
 (segment (start 50 23.37) (end 53.63 27) (width 0.5) (layer "F.Cu") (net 14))
 (segment (start 20.38 21.3) (end 22.18 19.5) (width 0.5) (layer "F.Cu") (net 14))
 (segment (start 42.905 14) (end 42.705 13.8) (width 0.5) (layer "F.Cu") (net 14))
 (segment (start 45 16.8) (end 42.46 16.8) (width 0.5) (layer "F.Cu") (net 14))
 (segment (start 22.18 19.5) (end 36.75 19.5) (width 0.5) (layer "F.Cu") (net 14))
 (segment (start 38.5 36.5) (end 33 42) (width 0.5) (layer "F.Cu") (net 14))
 (segment (start 50.219686 26.199) (end 52.829 26.199) (width 0.5) (layer "B.Cu") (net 14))
 (segment (start 40.66 36.5) (end 40.865 36.5) (width 0.5) (layer "B.Cu") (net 14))
 (segment (start 49.399 27.019686) (end 50.219686 26.199) (width 0.5) (layer "B.Cu") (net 14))
 (segment (start 52.829 26.199) (end 53.63 27) (width 0.5) (layer "B.Cu") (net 14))
 (segment (start 40.66 36.5) (end 40.834867 36.5) (width 0.5) (layer "B.Cu") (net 14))
 (segment (start 40.834867 36.5) (end 49.399 27.935867) (width 0.5) (layer "B.Cu") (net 14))
 (segment (start 49.399 27.935867) (end 49.399 27.019686) (width 0.5) (layer "B.Cu") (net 14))
 (segment (start 40.66 36.5) (end 41 36.5) (width 0.5) (layer "B.Cu") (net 14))
 (segment (start 46.5 37) (end 46.5 42) (width 0.5) (layer "F.Cu") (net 5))
 (segment (start 50 33.5) (end 46.5 37) (width 0.5) (layer "F.Cu") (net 5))
 (segment (start 32.3 16.8) (end 30.205 16.8) (width 0.5) (layer "F.Cu") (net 15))
 (segment (start 22.231 27.069) (end 20.38 28.92) (width 0.5) (layer "B.Cu") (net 15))
 (segment (start 22.231 24.616976) (end 22.231 27.069) (width 0.5) (layer "B.Cu") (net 15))
 (segment (start 22.231 24.616976) (end 30.047976 16.8) (width 0.5) (layer "B.Cu") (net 15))
 (segment (start 30.047976 16.8) (end 30.205 16.8) (width 0.5) (layer "B.Cu") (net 15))
 (segment (start 32.3 13.8) (end 30.205 13.8) (width 0.5) (layer "F.Cu") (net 2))
 (segment (start 32.3 13.8) (end 38.927182 13.8) (width 0.5) (layer "B.Cu") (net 2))
 (segment (start 54.139 17.349) (end 61.25 24.46) (width 0.5) (layer "B.Cu") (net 2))
 (segment (start 43.796976 15.349) (end 45.796976 17.349) (width 0.5) (layer "B.Cu") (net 2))
 (segment (start 38.927182 13.8) (end 40.476182 15.349) (width 0.5) (layer "B.Cu") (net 2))
 (segment (start 40.476182 15.349) (end 43.796976 15.349) (width 0.5) (layer "B.Cu") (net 2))
 (segment (start 45.796976 17.349) (end 54.139 17.349) (width 0.5) (layer "B.Cu") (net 2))
 (segment (start 52.42 34.12) (end 52.42 37.3) (width 0.5) (layer "F.Cu") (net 18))
 (segment (start 53.77 32.77) (end 52.42 34.12) (width 0.5) (layer "F.Cu") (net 18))
 (segment (start 60.549 38.201) (end 57.5 41.25) (width 0.5) (layer "F.Cu") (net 6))
 (segment (start 57.5 41.25) (end 57.5 43.58) (width 0.5) (layer "F.Cu") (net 6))
 (segment (start 64.25 37) (end 63.049 38.201) (width 0.5) (layer "F.Cu") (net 6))
 (segment (start 52.5 31.5) (end 58.75 31.5) (width 0.5) (layer "F.Cu") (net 6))
 (segment (start 63.049 38.201) (end 60.549 38.201) (width 0.5) (layer "F.Cu") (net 6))
 (segment (start 58.75 31.5) (end 64.25 37) (width 0.5) (layer "F.Cu") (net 6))
 (segment (start 30.705 36.5) (end 30.5 36.5) (width 0.5) (layer "F.Cu") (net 9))
 (segment (start 30.46 36.54) (end 30.5 36.5) (width 0.5) (layer "F.Cu") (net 9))
 (segment (start 29.5 40.6) (end 29.5 38.04) (width 0.5) (layer "F.Cu") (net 9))
 (segment (start 28.04 36.5) (end 28 36.54) (width 0.5) (layer "F.Cu") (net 9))
 (segment (start 19.378976 37.991) (end 26.549 37.991) (width 0.5) (layer "F.Cu") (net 9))
 (segment (start 26.549 37.991) (end 28 36.54) (width 0.5) (layer "F.Cu") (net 9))
 (segment (start 15 33.612024) (end 19.378976 37.991) (width 0.5) (layer "F.Cu") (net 9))
 (segment (start 30.84 36.635) (end 30.705 36.5) (width 0.5) (layer "F.Cu") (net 9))
 (segment (start 15 33.5) (end 15 33.612024) (width 0.5) (layer "F.Cu") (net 9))
 (segment (start 29.5 38.04) (end 28 36.54) (width 0.5) (layer "F.Cu") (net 9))
 (segment (start 28 36.54) (end 30.46 36.54) (width 0.5) (layer "F.Cu") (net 9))
 (via (at 29.5 40.6) (size 1.5) (drill 0.75) (layers "F.Cu" "B.Cu") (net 9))
 (segment (start 36.374 43.626) (end 32.5 43.626) (width 0.5) (layer "B.Cu") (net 9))
 (segment (start 38 42) (end 36.374 43.626) (width 0.5) (layer "B.Cu") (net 9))
 (segment (start 32.5 43.626) (end 32.378265 43.626) (width 0.5) (layer "B.Cu") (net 9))
 (segment (start 32.378265 43.626) (end 29.5 40.747735) (width 0.5) (layer "B.Cu") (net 9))
 (segment (start 29.5 40.747735) (end 29.5 40.6) (width 0.5) (layer "B.Cu") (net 9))
 (segment (start 42.374 43.626) (end 44 42) (width 0.5) (layer "F.Cu") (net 4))
 (segment (start 23.626 43.626) (end 42.374 43.626) (width 0.5) (layer "F.Cu") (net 4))
 (segment (start 22 42) (end 23.626 43.626) (width 0.5) (layer "F.Cu") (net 4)))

